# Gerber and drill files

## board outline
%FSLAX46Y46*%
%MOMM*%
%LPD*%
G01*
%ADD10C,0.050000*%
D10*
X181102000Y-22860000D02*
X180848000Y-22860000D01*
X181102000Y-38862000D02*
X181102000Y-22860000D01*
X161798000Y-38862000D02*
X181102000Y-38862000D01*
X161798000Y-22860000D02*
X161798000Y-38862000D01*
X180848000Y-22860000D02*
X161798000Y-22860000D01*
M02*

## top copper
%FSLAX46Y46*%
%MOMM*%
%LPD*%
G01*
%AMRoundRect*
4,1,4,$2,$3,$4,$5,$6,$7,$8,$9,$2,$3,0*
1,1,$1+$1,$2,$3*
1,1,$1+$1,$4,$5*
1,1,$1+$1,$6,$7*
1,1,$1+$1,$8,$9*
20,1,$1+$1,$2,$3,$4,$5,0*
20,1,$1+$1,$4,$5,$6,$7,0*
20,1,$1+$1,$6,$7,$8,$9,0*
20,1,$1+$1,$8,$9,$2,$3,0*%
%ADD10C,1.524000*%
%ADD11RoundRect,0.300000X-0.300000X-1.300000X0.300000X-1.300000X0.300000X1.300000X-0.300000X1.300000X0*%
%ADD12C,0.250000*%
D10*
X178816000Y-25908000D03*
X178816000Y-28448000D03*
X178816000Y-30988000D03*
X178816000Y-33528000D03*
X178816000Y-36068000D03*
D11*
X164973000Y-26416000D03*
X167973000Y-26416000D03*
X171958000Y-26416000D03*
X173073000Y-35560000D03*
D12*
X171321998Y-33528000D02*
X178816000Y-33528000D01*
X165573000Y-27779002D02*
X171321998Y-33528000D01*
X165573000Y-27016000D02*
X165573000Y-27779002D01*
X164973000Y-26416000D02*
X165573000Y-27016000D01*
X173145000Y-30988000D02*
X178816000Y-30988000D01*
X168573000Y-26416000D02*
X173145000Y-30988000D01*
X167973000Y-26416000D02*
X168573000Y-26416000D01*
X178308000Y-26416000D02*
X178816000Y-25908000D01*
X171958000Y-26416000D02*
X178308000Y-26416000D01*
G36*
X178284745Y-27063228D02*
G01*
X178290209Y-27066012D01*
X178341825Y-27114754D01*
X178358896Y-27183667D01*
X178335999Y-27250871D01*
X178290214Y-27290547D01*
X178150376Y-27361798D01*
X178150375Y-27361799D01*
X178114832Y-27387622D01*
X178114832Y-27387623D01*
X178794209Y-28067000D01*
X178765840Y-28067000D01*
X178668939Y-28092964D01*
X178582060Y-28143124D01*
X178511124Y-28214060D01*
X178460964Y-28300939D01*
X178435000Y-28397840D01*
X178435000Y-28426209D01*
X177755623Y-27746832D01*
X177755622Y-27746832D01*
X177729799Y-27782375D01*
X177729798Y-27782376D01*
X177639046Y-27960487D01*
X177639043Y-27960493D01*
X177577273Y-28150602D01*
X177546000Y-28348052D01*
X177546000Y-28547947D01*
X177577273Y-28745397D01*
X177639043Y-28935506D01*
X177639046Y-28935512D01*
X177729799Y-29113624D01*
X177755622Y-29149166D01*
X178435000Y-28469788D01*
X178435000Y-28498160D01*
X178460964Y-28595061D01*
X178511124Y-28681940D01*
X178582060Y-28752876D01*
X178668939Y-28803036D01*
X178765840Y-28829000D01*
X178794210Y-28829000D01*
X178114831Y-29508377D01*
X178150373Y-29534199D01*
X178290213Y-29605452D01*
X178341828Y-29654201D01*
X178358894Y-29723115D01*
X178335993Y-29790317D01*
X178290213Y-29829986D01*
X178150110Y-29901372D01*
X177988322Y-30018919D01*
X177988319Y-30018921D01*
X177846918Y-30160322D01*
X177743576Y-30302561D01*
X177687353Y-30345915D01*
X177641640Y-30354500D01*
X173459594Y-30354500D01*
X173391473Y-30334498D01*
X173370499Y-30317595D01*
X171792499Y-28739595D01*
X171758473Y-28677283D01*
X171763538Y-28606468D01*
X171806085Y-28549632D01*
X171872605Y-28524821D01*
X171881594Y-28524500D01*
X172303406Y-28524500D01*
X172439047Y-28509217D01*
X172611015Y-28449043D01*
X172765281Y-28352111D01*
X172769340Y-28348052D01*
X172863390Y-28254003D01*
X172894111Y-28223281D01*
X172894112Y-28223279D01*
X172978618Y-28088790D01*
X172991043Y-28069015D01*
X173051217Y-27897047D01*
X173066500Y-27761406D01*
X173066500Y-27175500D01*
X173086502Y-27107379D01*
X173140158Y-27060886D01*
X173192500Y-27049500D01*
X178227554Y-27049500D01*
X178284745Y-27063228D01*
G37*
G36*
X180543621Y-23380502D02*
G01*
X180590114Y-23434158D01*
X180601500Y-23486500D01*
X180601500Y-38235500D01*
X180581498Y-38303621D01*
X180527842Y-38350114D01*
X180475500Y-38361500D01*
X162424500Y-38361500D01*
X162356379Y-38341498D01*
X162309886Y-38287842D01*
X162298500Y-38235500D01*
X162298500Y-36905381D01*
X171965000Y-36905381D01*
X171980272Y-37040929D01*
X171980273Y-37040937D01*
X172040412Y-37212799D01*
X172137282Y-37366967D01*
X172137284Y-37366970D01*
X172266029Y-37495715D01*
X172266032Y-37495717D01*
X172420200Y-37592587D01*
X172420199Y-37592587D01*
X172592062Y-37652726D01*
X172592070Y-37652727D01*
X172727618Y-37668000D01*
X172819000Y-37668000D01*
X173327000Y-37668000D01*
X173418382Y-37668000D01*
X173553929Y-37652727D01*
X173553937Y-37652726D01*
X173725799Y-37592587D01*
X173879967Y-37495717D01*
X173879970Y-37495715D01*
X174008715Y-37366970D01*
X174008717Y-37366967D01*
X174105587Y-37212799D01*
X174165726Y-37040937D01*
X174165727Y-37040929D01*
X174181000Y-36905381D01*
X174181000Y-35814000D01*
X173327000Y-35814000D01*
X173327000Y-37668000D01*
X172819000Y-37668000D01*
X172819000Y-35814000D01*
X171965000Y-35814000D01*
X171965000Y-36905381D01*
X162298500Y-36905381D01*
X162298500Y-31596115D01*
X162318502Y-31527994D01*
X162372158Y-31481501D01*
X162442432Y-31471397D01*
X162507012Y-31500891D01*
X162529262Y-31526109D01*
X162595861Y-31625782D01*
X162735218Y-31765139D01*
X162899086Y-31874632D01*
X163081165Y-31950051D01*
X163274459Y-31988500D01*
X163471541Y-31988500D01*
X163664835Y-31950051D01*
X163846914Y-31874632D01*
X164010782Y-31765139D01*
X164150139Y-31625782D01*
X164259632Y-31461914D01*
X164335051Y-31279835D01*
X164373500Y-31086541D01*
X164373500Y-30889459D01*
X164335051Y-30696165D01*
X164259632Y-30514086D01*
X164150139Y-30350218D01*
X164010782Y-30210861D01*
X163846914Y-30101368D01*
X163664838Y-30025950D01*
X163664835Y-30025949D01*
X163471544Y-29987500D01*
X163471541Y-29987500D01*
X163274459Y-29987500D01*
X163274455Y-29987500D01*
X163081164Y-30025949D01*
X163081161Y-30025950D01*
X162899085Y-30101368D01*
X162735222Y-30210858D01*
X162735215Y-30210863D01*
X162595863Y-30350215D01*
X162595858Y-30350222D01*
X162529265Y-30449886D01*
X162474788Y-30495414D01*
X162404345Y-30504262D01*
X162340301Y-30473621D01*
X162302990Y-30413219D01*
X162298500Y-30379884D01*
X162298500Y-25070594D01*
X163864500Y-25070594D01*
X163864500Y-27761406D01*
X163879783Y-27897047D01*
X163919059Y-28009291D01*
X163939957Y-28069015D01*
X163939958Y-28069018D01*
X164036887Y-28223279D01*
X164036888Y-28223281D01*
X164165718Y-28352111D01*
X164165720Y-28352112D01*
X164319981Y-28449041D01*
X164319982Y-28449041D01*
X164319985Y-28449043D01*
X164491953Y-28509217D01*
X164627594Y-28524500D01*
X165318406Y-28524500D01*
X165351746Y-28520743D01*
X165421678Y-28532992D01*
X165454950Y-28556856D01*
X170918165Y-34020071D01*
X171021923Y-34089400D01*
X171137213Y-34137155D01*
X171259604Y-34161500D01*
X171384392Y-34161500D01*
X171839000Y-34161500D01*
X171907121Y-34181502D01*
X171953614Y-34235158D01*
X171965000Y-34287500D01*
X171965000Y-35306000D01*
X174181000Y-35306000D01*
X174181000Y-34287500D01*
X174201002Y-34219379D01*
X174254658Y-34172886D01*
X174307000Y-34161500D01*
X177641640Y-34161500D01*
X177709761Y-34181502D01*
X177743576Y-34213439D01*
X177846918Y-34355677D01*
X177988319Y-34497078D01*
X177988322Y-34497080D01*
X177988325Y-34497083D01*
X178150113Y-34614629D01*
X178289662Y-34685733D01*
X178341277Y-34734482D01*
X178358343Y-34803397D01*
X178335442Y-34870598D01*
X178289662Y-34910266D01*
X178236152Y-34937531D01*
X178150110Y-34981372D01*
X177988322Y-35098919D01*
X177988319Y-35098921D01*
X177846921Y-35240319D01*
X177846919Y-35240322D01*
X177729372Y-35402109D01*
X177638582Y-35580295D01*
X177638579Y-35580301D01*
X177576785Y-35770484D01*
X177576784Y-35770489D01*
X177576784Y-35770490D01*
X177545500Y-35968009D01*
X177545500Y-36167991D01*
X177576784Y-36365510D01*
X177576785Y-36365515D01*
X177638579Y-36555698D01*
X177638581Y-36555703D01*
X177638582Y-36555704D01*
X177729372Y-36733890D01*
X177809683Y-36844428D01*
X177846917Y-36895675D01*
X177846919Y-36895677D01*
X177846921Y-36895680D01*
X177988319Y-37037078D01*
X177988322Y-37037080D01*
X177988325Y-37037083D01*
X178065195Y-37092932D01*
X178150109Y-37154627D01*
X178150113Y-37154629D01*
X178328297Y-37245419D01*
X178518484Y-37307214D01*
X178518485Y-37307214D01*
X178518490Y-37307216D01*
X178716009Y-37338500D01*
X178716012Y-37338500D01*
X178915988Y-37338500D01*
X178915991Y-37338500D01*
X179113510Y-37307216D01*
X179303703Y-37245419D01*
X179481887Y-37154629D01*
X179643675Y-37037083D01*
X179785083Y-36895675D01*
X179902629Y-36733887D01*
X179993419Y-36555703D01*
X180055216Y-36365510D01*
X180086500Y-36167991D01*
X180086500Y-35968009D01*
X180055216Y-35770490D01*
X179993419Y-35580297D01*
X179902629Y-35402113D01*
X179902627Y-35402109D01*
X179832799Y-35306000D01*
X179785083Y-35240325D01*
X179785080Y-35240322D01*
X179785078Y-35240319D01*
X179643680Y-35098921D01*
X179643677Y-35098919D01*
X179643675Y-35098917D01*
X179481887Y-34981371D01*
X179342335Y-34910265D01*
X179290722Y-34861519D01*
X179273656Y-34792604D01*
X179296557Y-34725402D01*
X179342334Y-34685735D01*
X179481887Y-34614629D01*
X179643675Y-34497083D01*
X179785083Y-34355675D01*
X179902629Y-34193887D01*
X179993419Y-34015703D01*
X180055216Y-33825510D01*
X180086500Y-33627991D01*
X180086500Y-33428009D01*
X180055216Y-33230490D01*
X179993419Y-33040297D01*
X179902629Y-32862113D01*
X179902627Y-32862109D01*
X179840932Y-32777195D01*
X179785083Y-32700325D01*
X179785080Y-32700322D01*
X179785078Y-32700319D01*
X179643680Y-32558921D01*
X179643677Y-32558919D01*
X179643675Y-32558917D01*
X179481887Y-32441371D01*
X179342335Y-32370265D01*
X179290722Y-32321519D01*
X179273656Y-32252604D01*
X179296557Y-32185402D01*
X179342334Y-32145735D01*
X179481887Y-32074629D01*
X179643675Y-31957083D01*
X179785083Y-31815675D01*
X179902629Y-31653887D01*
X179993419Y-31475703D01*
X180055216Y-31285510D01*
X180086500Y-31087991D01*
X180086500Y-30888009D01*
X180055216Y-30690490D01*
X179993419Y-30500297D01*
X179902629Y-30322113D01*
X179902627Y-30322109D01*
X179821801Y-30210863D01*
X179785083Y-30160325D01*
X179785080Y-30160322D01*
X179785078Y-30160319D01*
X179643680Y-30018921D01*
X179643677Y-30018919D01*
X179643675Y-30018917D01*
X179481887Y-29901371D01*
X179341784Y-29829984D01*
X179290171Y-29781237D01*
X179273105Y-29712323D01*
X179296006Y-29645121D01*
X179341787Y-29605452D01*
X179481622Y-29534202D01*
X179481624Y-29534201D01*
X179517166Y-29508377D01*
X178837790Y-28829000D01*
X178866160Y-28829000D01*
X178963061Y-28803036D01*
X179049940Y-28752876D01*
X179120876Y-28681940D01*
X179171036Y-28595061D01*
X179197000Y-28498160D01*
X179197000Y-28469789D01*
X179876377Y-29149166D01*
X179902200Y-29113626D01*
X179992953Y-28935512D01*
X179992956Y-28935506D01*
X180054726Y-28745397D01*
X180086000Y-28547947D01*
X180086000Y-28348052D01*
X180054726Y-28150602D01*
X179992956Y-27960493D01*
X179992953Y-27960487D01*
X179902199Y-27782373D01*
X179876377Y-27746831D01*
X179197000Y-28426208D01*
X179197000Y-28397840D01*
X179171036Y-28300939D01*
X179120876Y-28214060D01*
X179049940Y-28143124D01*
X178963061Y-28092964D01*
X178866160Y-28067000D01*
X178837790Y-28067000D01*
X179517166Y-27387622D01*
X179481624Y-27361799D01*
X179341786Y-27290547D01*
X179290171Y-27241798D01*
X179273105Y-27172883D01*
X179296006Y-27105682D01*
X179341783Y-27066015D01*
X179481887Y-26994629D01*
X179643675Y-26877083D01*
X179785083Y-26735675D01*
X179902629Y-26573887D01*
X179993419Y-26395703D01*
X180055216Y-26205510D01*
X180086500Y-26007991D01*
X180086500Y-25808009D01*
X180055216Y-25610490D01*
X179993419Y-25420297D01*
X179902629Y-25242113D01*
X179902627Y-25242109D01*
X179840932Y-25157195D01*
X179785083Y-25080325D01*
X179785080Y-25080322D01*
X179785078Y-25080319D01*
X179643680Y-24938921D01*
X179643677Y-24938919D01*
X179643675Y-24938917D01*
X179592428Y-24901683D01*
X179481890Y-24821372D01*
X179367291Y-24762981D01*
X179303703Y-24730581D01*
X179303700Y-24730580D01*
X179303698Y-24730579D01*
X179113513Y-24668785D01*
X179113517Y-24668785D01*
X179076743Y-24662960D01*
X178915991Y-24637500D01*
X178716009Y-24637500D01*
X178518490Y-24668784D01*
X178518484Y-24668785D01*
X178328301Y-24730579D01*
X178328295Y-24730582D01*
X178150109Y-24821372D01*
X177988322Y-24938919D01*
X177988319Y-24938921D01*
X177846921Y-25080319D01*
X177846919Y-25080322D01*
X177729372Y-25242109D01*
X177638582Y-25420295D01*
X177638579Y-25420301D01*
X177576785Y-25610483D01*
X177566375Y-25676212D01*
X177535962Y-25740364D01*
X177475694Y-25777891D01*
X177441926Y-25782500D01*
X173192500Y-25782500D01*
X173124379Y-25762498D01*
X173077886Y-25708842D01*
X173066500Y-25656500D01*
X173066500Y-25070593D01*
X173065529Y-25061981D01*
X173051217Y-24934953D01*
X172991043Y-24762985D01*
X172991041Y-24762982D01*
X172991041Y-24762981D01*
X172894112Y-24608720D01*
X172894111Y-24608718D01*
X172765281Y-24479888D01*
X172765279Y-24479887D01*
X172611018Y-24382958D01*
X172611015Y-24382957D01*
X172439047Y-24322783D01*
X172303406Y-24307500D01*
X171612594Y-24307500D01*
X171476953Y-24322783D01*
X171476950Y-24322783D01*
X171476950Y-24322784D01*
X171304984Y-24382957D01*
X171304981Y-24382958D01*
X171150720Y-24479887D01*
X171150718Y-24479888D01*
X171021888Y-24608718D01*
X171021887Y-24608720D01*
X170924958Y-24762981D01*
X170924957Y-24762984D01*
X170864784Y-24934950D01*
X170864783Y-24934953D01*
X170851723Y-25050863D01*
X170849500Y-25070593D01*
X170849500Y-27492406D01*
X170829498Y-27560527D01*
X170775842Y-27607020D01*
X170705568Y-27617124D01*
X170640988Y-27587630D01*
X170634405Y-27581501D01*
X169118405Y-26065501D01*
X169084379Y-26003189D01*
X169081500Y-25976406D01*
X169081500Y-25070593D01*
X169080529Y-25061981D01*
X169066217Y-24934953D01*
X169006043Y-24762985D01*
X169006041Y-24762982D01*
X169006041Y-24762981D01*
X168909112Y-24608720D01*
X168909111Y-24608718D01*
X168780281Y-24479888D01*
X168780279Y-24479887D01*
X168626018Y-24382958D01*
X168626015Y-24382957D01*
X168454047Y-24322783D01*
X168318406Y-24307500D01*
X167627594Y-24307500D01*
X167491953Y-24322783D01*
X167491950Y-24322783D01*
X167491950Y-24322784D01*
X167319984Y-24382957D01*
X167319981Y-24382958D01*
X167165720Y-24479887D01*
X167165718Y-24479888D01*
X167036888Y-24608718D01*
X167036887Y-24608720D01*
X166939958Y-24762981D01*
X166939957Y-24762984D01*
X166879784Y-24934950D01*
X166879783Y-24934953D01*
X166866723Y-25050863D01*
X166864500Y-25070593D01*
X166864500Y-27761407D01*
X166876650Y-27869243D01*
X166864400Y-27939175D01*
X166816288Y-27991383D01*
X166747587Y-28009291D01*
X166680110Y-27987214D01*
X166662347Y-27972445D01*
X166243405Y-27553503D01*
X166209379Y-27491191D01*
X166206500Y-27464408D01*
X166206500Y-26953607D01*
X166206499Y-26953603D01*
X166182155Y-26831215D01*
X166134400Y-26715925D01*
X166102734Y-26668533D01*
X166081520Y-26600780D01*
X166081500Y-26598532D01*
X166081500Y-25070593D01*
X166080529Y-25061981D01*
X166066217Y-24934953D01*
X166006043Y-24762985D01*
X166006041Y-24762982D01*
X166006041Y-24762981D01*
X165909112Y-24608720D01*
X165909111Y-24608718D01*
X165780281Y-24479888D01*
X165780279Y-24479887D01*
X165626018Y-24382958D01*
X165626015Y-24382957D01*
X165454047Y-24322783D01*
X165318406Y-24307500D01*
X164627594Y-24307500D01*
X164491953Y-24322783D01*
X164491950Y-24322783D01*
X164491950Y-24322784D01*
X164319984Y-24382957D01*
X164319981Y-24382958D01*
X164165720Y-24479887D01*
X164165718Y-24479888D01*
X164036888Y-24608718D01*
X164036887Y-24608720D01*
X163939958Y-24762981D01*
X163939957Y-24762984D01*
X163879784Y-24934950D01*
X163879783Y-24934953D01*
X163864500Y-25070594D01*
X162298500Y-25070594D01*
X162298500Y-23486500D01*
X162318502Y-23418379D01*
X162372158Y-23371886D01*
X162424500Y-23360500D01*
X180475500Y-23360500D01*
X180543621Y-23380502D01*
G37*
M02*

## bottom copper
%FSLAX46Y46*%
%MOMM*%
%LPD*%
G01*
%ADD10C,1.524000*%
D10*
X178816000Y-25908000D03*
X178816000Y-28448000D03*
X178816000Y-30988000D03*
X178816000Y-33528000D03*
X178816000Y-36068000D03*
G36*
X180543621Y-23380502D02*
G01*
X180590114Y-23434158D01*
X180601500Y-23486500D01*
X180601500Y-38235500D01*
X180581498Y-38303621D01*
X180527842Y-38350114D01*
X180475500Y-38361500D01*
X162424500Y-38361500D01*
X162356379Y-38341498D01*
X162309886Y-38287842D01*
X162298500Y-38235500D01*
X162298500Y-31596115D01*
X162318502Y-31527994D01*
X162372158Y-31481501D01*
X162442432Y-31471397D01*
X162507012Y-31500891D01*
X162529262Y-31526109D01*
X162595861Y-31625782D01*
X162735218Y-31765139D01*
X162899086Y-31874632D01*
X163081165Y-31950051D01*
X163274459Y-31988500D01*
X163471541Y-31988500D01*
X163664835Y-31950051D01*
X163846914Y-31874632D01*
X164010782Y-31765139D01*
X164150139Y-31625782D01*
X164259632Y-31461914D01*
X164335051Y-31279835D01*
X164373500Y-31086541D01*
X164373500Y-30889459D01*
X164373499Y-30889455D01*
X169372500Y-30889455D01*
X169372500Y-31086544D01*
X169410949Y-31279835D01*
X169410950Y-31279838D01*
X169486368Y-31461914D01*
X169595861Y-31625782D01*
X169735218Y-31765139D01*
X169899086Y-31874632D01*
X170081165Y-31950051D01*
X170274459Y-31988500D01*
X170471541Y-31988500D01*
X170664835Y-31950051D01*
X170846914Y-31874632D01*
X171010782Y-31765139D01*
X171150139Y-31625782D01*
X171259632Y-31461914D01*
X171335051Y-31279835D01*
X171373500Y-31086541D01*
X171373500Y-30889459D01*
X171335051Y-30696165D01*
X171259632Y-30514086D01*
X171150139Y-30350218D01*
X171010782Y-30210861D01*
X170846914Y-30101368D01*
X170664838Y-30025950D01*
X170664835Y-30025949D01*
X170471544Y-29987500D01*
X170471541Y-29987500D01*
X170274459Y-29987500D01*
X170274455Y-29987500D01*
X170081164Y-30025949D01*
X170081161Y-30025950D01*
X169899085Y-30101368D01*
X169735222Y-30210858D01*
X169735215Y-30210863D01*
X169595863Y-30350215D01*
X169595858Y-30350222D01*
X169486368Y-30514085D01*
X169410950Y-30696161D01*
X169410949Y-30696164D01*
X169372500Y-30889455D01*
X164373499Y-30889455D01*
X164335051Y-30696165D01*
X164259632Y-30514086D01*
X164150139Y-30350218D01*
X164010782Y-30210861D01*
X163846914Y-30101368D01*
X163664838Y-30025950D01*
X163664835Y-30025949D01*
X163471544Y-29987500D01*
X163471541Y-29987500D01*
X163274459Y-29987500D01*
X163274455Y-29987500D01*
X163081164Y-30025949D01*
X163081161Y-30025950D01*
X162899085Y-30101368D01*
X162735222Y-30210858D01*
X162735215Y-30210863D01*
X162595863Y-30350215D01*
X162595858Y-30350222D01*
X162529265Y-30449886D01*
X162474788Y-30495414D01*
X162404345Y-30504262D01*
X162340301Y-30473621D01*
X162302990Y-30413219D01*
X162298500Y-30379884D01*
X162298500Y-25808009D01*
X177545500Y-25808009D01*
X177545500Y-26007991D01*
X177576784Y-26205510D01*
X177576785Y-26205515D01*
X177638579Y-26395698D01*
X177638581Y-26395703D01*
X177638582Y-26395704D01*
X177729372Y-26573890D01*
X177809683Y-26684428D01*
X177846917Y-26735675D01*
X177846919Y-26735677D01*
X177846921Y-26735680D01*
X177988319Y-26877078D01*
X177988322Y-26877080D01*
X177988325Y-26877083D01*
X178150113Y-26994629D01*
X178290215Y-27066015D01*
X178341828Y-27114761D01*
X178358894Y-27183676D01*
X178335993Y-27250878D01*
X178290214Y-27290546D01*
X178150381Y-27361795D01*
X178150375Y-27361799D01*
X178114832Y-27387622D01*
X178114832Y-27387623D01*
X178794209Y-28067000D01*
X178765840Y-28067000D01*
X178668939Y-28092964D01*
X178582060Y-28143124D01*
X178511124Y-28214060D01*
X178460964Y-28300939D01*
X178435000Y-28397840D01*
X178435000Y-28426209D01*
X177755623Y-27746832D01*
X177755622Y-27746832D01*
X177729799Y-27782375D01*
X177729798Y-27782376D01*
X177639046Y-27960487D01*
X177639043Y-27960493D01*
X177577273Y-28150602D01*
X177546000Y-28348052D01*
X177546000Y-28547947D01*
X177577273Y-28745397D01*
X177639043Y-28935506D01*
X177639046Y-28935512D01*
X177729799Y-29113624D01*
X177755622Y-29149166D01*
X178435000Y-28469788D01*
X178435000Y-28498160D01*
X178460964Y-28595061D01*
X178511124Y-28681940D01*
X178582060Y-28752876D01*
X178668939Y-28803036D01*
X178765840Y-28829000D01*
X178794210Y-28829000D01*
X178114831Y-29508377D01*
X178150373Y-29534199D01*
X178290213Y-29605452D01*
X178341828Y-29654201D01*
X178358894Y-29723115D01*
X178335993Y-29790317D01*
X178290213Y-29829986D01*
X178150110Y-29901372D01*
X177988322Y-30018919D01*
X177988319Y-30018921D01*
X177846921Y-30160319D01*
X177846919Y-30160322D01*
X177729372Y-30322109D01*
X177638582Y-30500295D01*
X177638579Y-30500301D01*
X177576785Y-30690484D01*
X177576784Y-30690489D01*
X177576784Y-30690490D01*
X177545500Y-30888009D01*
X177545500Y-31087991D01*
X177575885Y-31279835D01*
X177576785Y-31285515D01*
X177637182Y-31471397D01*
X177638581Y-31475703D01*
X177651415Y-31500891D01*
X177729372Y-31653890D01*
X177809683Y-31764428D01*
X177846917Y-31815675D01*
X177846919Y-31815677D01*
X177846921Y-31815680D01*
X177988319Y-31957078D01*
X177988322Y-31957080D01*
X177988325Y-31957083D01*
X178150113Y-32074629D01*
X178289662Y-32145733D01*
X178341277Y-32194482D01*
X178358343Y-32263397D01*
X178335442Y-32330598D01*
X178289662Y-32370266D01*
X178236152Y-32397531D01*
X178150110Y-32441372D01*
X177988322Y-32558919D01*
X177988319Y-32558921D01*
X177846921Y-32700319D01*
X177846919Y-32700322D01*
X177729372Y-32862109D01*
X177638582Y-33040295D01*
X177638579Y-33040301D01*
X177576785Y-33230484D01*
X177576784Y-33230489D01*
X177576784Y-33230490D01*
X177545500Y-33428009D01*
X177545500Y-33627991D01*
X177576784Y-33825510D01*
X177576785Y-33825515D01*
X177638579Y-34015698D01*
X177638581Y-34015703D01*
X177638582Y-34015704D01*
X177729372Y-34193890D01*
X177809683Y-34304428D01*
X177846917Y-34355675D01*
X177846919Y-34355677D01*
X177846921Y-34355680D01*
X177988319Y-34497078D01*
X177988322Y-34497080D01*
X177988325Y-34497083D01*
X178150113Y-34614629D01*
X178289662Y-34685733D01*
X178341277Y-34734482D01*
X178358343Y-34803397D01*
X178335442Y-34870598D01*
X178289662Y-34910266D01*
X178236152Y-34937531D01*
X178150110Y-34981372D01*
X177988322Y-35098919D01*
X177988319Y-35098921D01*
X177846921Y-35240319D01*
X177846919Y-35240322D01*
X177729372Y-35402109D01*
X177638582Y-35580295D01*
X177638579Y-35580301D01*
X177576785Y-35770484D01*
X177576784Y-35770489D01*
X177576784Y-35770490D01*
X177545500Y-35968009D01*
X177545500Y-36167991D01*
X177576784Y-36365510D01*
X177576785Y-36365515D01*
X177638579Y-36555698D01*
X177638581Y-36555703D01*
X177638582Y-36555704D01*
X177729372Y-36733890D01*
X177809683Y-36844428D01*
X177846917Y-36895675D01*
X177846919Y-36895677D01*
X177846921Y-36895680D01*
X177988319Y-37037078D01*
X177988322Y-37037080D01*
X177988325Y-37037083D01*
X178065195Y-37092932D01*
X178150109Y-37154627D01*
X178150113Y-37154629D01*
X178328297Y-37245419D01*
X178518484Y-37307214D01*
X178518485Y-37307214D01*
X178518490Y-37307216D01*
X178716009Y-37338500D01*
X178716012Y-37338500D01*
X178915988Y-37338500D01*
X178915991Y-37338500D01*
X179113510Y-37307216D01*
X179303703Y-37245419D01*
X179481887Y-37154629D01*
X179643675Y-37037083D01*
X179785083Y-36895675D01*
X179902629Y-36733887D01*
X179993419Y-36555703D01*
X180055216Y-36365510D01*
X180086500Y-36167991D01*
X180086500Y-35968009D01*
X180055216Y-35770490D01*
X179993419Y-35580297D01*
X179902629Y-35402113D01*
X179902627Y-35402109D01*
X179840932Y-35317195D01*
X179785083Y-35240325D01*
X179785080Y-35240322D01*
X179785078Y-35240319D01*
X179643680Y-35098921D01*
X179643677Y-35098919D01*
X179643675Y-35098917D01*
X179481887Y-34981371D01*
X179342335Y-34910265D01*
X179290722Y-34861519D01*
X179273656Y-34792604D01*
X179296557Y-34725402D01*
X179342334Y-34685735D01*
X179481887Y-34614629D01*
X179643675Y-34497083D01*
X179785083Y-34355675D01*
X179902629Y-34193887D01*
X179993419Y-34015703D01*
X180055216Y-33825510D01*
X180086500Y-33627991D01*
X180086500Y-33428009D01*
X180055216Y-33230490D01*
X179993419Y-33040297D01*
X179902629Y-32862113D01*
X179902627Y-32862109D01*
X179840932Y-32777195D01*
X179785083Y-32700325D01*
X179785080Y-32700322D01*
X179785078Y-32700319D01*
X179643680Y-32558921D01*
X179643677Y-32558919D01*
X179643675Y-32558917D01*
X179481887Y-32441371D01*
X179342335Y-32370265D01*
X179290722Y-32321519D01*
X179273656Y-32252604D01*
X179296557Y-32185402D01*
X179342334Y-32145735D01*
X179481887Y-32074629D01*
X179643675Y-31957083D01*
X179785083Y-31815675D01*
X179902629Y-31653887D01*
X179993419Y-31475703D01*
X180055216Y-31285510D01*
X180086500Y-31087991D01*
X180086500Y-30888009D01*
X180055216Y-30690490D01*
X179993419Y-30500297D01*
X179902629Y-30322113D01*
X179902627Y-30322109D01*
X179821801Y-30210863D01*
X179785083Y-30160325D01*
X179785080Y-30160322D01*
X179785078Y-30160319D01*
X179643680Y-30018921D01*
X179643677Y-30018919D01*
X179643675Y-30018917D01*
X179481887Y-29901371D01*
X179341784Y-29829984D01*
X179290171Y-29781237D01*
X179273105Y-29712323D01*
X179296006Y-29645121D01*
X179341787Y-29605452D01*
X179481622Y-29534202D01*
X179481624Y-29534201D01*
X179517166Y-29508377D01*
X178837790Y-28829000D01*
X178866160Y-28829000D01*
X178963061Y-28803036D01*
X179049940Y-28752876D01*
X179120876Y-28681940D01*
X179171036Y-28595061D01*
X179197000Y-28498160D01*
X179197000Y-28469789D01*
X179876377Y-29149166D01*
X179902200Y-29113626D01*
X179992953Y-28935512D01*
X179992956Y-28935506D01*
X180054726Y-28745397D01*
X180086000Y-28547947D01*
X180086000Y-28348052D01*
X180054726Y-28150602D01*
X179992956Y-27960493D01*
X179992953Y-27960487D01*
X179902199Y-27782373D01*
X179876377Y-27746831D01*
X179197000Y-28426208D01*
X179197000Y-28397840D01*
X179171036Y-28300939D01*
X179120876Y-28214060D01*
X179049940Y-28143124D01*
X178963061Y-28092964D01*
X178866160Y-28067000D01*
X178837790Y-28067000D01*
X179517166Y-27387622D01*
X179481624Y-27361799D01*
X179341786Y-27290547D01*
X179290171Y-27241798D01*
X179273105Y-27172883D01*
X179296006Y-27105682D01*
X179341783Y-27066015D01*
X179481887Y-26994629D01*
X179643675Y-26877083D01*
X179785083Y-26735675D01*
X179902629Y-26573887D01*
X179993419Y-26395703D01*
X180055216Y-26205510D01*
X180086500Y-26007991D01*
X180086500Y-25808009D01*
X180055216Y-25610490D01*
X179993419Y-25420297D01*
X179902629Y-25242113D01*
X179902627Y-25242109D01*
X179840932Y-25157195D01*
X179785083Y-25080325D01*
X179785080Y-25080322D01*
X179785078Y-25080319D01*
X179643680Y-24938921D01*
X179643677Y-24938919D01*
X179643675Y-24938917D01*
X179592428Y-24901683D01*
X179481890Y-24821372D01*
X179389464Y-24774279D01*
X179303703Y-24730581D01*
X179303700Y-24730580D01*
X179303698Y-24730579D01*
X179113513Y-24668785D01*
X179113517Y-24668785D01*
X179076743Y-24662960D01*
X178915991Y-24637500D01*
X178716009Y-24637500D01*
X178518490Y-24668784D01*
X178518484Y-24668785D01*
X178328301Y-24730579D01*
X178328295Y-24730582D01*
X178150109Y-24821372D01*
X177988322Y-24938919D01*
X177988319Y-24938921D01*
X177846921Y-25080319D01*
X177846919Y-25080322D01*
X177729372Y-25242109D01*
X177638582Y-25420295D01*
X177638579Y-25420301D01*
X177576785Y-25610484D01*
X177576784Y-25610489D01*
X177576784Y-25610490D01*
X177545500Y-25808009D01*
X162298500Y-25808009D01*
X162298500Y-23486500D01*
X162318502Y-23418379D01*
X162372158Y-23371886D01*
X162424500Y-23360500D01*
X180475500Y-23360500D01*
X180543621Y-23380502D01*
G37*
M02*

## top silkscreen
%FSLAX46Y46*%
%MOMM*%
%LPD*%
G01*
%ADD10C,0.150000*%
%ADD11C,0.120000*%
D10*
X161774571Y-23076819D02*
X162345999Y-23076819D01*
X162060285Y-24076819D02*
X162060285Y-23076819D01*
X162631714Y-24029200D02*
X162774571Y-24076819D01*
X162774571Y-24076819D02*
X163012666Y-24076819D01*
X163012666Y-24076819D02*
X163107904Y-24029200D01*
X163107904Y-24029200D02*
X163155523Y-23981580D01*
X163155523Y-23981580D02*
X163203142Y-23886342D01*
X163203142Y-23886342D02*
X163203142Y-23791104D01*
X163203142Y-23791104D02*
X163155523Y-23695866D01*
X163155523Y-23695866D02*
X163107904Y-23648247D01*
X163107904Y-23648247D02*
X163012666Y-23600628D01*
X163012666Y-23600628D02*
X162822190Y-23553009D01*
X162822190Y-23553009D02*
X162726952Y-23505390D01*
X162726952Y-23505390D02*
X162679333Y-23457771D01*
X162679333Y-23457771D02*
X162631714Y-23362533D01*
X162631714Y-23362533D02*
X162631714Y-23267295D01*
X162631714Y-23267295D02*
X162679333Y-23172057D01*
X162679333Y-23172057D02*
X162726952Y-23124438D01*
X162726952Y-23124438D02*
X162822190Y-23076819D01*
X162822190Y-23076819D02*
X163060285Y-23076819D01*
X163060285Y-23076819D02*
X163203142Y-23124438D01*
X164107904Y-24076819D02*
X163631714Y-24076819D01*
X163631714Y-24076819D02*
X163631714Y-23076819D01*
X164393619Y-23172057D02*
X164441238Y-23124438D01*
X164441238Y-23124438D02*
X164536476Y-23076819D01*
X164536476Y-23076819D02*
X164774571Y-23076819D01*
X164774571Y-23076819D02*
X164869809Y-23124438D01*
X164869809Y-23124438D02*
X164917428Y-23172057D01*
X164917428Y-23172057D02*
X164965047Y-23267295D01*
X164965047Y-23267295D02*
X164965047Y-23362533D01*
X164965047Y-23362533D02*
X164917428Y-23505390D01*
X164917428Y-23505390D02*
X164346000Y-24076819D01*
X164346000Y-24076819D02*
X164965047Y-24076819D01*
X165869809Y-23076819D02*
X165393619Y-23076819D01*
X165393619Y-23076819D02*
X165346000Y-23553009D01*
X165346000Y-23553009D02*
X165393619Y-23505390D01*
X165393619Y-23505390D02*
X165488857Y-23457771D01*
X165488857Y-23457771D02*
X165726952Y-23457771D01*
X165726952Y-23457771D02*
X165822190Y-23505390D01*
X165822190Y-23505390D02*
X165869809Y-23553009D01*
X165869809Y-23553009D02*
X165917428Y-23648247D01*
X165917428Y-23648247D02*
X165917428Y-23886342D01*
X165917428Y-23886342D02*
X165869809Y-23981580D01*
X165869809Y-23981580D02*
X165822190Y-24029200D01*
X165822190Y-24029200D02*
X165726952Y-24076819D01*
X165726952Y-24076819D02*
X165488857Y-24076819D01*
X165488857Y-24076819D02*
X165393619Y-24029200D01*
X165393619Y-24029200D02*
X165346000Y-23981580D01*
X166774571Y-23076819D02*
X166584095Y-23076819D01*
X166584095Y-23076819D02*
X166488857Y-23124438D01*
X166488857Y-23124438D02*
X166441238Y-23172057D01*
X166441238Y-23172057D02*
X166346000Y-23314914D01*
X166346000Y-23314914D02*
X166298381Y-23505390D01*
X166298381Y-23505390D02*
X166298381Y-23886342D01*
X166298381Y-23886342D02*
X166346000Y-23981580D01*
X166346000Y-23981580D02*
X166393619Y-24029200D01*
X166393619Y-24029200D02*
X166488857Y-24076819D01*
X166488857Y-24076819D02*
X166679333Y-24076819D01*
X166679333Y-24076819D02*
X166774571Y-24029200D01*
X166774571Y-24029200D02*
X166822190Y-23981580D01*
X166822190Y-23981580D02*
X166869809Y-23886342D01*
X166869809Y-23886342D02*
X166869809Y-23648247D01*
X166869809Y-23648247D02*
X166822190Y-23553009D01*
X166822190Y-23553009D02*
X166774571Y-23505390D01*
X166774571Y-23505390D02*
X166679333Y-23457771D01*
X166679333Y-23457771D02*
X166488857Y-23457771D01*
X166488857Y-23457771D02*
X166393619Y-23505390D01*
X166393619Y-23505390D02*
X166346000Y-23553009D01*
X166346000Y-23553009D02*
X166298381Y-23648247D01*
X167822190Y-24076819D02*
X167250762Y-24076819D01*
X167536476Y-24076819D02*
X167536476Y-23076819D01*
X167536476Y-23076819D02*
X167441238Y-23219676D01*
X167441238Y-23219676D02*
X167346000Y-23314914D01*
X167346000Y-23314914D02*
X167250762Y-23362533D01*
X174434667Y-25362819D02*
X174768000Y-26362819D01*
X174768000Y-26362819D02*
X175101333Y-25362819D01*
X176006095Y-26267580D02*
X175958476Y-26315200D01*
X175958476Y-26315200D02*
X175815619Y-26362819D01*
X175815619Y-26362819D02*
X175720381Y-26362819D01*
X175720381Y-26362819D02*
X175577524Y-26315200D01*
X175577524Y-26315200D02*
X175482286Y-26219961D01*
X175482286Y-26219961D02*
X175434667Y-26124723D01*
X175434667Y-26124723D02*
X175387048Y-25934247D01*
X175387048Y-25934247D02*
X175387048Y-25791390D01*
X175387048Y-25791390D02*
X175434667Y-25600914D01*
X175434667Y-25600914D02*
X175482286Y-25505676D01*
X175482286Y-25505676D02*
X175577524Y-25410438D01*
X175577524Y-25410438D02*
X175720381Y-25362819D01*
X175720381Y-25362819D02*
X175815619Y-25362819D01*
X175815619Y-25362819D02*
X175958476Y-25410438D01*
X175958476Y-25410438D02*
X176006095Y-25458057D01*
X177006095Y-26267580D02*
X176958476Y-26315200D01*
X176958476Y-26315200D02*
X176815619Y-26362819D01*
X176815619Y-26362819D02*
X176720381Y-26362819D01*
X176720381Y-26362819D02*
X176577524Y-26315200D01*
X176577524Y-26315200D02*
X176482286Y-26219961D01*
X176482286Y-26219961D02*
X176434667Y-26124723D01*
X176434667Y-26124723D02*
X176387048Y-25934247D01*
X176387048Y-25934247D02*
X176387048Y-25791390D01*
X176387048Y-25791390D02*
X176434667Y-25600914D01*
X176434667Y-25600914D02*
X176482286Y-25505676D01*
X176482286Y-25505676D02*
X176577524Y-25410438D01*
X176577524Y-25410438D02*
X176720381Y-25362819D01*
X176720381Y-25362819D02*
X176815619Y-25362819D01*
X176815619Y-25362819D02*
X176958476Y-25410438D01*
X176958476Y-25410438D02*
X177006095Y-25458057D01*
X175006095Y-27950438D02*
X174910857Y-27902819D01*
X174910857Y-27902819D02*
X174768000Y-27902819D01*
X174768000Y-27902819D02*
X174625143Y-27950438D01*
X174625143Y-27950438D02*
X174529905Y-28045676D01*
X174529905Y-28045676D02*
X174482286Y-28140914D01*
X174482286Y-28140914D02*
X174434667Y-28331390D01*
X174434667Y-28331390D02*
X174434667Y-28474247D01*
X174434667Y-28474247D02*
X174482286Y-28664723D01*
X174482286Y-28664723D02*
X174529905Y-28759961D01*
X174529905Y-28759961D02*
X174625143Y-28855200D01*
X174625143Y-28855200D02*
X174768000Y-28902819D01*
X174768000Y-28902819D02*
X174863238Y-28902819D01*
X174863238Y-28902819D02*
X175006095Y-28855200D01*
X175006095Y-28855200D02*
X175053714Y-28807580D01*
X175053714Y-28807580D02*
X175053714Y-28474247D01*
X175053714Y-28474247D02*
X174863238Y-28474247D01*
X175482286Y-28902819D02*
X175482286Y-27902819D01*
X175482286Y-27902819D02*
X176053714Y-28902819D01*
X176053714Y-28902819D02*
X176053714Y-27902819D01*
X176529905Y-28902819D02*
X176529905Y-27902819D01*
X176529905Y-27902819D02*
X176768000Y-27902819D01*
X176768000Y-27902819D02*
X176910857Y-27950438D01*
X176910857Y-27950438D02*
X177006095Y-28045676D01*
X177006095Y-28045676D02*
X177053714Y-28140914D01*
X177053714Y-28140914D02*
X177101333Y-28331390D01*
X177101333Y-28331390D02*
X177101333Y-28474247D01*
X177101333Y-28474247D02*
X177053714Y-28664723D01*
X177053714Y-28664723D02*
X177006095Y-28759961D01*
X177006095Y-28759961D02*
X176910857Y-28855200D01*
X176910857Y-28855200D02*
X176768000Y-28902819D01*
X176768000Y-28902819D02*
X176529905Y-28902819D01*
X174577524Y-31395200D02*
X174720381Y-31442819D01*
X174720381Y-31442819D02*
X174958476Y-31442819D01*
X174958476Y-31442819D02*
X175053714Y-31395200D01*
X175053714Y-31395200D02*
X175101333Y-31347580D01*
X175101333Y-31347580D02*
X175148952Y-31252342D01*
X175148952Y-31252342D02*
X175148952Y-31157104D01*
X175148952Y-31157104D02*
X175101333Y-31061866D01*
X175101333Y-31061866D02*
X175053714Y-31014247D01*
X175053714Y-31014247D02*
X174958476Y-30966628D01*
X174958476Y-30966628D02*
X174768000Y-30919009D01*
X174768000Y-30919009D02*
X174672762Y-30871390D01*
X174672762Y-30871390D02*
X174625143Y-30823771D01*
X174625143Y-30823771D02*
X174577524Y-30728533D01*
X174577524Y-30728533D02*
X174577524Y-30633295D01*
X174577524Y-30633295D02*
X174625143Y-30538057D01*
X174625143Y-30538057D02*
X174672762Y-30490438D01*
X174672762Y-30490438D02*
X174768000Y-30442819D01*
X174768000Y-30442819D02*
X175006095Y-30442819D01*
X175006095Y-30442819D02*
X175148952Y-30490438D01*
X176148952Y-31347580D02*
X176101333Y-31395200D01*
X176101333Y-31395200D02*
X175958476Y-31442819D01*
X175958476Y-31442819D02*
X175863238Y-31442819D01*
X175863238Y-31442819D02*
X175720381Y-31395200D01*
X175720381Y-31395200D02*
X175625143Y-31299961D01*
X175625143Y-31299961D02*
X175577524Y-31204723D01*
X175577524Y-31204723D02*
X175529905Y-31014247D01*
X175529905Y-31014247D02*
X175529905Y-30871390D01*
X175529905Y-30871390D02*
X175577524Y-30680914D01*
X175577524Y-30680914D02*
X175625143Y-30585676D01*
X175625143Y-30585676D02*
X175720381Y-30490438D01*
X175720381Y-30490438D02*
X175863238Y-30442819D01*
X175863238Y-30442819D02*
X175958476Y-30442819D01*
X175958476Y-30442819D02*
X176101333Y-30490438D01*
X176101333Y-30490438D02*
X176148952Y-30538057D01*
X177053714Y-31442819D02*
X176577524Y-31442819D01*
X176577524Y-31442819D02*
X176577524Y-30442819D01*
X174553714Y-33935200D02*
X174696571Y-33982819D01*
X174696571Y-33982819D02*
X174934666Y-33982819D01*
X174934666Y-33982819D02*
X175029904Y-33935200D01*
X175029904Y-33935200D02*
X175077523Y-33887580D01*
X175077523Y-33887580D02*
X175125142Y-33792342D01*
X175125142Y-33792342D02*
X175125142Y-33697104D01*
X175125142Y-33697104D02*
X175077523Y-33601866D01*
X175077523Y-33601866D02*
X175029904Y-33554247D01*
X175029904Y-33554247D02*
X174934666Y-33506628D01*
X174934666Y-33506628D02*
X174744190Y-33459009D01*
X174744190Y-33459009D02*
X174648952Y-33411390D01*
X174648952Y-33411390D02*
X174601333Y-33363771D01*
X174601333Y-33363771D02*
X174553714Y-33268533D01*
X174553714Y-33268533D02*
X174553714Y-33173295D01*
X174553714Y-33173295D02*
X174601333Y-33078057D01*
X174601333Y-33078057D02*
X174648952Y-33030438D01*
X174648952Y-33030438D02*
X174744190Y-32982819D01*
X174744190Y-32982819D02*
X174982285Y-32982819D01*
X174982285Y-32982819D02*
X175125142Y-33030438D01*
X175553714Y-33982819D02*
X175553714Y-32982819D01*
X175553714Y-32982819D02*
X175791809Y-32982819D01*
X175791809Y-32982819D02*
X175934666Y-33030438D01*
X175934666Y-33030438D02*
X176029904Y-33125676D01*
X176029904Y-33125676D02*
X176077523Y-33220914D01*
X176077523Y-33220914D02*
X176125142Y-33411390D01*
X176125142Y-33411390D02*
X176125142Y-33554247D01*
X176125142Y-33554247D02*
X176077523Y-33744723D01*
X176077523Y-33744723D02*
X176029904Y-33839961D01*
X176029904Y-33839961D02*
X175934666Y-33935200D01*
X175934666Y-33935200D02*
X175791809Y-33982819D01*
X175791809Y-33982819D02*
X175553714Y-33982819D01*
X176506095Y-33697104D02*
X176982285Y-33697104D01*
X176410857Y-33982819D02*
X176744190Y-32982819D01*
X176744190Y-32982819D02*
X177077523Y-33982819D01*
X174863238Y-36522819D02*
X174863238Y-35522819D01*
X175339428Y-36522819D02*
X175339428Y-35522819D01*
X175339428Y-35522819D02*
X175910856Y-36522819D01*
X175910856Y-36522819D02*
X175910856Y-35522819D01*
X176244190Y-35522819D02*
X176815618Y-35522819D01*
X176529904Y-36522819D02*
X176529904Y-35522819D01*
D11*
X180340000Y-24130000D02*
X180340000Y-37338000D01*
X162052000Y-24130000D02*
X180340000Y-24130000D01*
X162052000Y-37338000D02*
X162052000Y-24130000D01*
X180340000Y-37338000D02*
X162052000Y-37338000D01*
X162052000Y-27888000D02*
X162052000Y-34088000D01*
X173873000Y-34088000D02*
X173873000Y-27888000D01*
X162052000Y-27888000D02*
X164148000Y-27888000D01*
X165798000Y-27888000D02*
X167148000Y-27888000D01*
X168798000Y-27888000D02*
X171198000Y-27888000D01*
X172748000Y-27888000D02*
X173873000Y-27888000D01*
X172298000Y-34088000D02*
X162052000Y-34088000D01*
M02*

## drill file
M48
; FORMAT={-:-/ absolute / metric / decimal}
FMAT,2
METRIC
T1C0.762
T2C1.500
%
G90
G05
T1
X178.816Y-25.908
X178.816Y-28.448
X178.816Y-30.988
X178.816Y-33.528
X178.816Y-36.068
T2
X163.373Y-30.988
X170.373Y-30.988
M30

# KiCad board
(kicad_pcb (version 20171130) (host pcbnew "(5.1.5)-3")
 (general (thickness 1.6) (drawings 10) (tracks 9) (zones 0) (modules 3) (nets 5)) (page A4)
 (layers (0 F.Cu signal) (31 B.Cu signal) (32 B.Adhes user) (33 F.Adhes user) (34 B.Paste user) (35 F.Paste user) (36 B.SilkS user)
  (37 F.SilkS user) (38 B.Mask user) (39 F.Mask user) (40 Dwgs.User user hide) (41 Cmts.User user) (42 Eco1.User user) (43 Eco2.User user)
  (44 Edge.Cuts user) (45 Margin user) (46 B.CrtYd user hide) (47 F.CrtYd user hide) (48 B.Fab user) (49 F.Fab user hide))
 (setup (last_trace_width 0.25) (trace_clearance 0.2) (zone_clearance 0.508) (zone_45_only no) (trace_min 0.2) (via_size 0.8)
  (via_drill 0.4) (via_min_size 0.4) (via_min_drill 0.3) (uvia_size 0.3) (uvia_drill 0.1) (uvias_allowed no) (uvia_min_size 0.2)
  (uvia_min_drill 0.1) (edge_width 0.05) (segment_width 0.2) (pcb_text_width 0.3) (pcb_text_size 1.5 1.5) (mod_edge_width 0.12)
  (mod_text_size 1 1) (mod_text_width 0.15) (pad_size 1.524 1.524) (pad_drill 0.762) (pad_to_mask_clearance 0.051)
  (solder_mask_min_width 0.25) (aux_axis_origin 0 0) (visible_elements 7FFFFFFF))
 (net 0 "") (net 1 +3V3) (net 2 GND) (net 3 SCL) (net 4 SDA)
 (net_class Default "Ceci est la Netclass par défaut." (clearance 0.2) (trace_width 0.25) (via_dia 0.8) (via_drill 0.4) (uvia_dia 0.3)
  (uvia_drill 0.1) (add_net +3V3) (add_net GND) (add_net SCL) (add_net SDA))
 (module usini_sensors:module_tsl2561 (layer F.Cu) (at 178.816 25.908 180)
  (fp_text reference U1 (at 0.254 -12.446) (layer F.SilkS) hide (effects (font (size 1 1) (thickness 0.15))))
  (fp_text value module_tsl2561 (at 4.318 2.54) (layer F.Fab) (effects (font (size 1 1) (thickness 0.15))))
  (fp_line (start -1.524 1.778) (end -1.524 -11.43) (layer F.SilkS) (width 0.12))
  (fp_line (start 16.764 1.778) (end -1.524 1.778) (layer F.SilkS) (width 0.12))
  (fp_line (start 16.764 -11.43) (end 16.764 1.778) (layer F.SilkS) (width 0.12))
  (fp_line (start -1.524 -11.43) (end 16.764 -11.43) (layer F.SilkS) (width 0.12))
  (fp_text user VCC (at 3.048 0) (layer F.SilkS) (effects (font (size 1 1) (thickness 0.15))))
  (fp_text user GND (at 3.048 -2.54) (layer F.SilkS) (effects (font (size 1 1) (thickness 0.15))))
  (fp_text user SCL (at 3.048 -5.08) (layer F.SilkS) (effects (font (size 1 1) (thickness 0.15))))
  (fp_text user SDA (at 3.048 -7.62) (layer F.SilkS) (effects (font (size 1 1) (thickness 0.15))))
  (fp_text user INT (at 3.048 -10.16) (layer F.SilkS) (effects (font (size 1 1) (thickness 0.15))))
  (pad 5 thru_hole circle (at 0 0 180) (size 1.524 1.524) (drill 0.762) (layers *.Cu *.Mask) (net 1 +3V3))
  (pad 4 thru_hole circle (at 0 -2.54 180) (size 1.524 1.524) (drill 0.762) (layers *.Cu *.Mask) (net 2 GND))
  (pad 3 thru_hole circle (at 0 -5.08 180) (size 1.524 1.524) (drill 0.762) (layers *.Cu *.Mask) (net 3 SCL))
  (pad 2 thru_hole circle (at 0 -7.62 180) (size 1.524 1.524) (drill 0.762) (layers *.Cu *.Mask) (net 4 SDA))
  (pad 1 thru_hole circle (at 0 -10.16 180) (size 1.524 1.524) (drill 0.762) (layers *.Cu *.Mask)))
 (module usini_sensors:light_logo (layer B.Cu) (at 173.736 34.544)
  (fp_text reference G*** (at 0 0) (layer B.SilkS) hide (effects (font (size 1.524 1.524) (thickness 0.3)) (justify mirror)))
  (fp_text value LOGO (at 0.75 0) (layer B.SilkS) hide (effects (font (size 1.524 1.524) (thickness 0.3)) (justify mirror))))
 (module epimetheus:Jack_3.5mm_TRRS (layer F.Cu) (at 168.148 30.988)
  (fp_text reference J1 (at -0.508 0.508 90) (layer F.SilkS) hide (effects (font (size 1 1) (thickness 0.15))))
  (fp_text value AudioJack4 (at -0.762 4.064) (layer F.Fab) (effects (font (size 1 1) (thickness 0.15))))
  (fp_line (start -6.096 -3.1) (end -6.096 3.1) (layer F.SilkS) (width 0.12))
  (fp_line (start 5.725 3.1) (end 5.725 -3.1) (layer F.SilkS) (width 0.12))
  (fp_line (start -6.096 -3.1) (end -4 -3.1) (layer F.SilkS) (width 0.12))
  (fp_line (start -2.35 -3.1) (end -1 -3.1) (layer F.SilkS) (width 0.12))
  (fp_line (start 0.65 -3.1) (end 3.05 -3.1) (layer F.SilkS) (width 0.12))
  (fp_line (start 4.6 -3.1) (end 5.725 -3.1) (layer F.SilkS) (width 0.12))
  (fp_line (start 4.15 3.1) (end -6.096 3.1) (layer F.SilkS) (width 0.12))
  (pad "" np_thru_hole circle (at 2.225 0) (size 1.5 1.5) (drill 1.5) (layers *.Cu *.Mask))
  (pad "" np_thru_hole circle (at -4.775 0) (size 1.5 1.5) (drill 1.5) (layers *.Cu *.Mask))
  (pad R2 smd roundrect (at -3.175 -4.572) (size 1.2 3.2) (layers F.Cu F.Paste F.Mask) (roundrect_rratio 0.25) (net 4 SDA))
  (pad R1 smd roundrect (at -0.175 -4.572) (size 1.2 3.2) (layers F.Cu F.Paste F.Mask) (roundrect_rratio 0.25) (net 3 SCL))
  (pad T smd roundrect (at 3.81 -4.572) (size 1.2 3.2) (layers F.Cu F.Paste F.Mask) (roundrect_rratio 0.25) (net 1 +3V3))
  (pad S smd roundrect (at 4.925 4.572) (size 1.2 3.2) (layers F.Cu F.Paste F.Mask) (roundrect_rratio 0.25) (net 2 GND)))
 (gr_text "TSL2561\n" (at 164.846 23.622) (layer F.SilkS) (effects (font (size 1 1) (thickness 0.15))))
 (gr_line (start 181.102 22.86) (end 180.848 22.86) (layer Edge.Cuts) (width 0.05))
 (gr_line (start 181.102 38.862) (end 181.102 22.86) (layer Edge.Cuts) (width 0.05))
 (gr_line (start 161.798 38.862) (end 181.102 38.862) (layer Edge.Cuts) (width 0.05))
 (gr_line (start 161.798 22.86) (end 161.798 38.862) (layer Edge.Cuts) (width 0.05))
 (gr_line (start 180.848 22.86) (end 161.798 22.86) (layer Edge.Cuts) (width 0.05))
 (segment (start 171.321998 33.528) (end 178.816 33.528) (width 0.25) (layer F.Cu) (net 4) (status 20))
 (segment (start 165.573 27.779002) (end 171.321998 33.528) (width 0.25) (layer F.Cu) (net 4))
 (segment (start 165.573 27.016) (end 165.573 27.779002) (width 0.25) (layer F.Cu) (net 4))
 (segment (start 164.973 26.416) (end 165.573 27.016) (width 0.25) (layer F.Cu) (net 4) (status 10))
 (segment (start 173.145 30.988) (end 178.816 30.988) (width 0.25) (layer F.Cu) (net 3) (status 20))
 (segment (start 168.573 26.416) (end 173.145 30.988) (width 0.25) (layer F.Cu) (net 3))
 (segment (start 167.973 26.416) (end 168.573 26.416) (width 0.25) (layer F.Cu) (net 3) (status 10))
 (segment (start 178.308 26.416) (end 178.816 25.908) (width 0.25) (layer F.Cu) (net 1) (status 30))
 (segment (start 171.958 26.416) (end 178.308 26.416) (width 0.25) (layer F.Cu) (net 1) (status 30))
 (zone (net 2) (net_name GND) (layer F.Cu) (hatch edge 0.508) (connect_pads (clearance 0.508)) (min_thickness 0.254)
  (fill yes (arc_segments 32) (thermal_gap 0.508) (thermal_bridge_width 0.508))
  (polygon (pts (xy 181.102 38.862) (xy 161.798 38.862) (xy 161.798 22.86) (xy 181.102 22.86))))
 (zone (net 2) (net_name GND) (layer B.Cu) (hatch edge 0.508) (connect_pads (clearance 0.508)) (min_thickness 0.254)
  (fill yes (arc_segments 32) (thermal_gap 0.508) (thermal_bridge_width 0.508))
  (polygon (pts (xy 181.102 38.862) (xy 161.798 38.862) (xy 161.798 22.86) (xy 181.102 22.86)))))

